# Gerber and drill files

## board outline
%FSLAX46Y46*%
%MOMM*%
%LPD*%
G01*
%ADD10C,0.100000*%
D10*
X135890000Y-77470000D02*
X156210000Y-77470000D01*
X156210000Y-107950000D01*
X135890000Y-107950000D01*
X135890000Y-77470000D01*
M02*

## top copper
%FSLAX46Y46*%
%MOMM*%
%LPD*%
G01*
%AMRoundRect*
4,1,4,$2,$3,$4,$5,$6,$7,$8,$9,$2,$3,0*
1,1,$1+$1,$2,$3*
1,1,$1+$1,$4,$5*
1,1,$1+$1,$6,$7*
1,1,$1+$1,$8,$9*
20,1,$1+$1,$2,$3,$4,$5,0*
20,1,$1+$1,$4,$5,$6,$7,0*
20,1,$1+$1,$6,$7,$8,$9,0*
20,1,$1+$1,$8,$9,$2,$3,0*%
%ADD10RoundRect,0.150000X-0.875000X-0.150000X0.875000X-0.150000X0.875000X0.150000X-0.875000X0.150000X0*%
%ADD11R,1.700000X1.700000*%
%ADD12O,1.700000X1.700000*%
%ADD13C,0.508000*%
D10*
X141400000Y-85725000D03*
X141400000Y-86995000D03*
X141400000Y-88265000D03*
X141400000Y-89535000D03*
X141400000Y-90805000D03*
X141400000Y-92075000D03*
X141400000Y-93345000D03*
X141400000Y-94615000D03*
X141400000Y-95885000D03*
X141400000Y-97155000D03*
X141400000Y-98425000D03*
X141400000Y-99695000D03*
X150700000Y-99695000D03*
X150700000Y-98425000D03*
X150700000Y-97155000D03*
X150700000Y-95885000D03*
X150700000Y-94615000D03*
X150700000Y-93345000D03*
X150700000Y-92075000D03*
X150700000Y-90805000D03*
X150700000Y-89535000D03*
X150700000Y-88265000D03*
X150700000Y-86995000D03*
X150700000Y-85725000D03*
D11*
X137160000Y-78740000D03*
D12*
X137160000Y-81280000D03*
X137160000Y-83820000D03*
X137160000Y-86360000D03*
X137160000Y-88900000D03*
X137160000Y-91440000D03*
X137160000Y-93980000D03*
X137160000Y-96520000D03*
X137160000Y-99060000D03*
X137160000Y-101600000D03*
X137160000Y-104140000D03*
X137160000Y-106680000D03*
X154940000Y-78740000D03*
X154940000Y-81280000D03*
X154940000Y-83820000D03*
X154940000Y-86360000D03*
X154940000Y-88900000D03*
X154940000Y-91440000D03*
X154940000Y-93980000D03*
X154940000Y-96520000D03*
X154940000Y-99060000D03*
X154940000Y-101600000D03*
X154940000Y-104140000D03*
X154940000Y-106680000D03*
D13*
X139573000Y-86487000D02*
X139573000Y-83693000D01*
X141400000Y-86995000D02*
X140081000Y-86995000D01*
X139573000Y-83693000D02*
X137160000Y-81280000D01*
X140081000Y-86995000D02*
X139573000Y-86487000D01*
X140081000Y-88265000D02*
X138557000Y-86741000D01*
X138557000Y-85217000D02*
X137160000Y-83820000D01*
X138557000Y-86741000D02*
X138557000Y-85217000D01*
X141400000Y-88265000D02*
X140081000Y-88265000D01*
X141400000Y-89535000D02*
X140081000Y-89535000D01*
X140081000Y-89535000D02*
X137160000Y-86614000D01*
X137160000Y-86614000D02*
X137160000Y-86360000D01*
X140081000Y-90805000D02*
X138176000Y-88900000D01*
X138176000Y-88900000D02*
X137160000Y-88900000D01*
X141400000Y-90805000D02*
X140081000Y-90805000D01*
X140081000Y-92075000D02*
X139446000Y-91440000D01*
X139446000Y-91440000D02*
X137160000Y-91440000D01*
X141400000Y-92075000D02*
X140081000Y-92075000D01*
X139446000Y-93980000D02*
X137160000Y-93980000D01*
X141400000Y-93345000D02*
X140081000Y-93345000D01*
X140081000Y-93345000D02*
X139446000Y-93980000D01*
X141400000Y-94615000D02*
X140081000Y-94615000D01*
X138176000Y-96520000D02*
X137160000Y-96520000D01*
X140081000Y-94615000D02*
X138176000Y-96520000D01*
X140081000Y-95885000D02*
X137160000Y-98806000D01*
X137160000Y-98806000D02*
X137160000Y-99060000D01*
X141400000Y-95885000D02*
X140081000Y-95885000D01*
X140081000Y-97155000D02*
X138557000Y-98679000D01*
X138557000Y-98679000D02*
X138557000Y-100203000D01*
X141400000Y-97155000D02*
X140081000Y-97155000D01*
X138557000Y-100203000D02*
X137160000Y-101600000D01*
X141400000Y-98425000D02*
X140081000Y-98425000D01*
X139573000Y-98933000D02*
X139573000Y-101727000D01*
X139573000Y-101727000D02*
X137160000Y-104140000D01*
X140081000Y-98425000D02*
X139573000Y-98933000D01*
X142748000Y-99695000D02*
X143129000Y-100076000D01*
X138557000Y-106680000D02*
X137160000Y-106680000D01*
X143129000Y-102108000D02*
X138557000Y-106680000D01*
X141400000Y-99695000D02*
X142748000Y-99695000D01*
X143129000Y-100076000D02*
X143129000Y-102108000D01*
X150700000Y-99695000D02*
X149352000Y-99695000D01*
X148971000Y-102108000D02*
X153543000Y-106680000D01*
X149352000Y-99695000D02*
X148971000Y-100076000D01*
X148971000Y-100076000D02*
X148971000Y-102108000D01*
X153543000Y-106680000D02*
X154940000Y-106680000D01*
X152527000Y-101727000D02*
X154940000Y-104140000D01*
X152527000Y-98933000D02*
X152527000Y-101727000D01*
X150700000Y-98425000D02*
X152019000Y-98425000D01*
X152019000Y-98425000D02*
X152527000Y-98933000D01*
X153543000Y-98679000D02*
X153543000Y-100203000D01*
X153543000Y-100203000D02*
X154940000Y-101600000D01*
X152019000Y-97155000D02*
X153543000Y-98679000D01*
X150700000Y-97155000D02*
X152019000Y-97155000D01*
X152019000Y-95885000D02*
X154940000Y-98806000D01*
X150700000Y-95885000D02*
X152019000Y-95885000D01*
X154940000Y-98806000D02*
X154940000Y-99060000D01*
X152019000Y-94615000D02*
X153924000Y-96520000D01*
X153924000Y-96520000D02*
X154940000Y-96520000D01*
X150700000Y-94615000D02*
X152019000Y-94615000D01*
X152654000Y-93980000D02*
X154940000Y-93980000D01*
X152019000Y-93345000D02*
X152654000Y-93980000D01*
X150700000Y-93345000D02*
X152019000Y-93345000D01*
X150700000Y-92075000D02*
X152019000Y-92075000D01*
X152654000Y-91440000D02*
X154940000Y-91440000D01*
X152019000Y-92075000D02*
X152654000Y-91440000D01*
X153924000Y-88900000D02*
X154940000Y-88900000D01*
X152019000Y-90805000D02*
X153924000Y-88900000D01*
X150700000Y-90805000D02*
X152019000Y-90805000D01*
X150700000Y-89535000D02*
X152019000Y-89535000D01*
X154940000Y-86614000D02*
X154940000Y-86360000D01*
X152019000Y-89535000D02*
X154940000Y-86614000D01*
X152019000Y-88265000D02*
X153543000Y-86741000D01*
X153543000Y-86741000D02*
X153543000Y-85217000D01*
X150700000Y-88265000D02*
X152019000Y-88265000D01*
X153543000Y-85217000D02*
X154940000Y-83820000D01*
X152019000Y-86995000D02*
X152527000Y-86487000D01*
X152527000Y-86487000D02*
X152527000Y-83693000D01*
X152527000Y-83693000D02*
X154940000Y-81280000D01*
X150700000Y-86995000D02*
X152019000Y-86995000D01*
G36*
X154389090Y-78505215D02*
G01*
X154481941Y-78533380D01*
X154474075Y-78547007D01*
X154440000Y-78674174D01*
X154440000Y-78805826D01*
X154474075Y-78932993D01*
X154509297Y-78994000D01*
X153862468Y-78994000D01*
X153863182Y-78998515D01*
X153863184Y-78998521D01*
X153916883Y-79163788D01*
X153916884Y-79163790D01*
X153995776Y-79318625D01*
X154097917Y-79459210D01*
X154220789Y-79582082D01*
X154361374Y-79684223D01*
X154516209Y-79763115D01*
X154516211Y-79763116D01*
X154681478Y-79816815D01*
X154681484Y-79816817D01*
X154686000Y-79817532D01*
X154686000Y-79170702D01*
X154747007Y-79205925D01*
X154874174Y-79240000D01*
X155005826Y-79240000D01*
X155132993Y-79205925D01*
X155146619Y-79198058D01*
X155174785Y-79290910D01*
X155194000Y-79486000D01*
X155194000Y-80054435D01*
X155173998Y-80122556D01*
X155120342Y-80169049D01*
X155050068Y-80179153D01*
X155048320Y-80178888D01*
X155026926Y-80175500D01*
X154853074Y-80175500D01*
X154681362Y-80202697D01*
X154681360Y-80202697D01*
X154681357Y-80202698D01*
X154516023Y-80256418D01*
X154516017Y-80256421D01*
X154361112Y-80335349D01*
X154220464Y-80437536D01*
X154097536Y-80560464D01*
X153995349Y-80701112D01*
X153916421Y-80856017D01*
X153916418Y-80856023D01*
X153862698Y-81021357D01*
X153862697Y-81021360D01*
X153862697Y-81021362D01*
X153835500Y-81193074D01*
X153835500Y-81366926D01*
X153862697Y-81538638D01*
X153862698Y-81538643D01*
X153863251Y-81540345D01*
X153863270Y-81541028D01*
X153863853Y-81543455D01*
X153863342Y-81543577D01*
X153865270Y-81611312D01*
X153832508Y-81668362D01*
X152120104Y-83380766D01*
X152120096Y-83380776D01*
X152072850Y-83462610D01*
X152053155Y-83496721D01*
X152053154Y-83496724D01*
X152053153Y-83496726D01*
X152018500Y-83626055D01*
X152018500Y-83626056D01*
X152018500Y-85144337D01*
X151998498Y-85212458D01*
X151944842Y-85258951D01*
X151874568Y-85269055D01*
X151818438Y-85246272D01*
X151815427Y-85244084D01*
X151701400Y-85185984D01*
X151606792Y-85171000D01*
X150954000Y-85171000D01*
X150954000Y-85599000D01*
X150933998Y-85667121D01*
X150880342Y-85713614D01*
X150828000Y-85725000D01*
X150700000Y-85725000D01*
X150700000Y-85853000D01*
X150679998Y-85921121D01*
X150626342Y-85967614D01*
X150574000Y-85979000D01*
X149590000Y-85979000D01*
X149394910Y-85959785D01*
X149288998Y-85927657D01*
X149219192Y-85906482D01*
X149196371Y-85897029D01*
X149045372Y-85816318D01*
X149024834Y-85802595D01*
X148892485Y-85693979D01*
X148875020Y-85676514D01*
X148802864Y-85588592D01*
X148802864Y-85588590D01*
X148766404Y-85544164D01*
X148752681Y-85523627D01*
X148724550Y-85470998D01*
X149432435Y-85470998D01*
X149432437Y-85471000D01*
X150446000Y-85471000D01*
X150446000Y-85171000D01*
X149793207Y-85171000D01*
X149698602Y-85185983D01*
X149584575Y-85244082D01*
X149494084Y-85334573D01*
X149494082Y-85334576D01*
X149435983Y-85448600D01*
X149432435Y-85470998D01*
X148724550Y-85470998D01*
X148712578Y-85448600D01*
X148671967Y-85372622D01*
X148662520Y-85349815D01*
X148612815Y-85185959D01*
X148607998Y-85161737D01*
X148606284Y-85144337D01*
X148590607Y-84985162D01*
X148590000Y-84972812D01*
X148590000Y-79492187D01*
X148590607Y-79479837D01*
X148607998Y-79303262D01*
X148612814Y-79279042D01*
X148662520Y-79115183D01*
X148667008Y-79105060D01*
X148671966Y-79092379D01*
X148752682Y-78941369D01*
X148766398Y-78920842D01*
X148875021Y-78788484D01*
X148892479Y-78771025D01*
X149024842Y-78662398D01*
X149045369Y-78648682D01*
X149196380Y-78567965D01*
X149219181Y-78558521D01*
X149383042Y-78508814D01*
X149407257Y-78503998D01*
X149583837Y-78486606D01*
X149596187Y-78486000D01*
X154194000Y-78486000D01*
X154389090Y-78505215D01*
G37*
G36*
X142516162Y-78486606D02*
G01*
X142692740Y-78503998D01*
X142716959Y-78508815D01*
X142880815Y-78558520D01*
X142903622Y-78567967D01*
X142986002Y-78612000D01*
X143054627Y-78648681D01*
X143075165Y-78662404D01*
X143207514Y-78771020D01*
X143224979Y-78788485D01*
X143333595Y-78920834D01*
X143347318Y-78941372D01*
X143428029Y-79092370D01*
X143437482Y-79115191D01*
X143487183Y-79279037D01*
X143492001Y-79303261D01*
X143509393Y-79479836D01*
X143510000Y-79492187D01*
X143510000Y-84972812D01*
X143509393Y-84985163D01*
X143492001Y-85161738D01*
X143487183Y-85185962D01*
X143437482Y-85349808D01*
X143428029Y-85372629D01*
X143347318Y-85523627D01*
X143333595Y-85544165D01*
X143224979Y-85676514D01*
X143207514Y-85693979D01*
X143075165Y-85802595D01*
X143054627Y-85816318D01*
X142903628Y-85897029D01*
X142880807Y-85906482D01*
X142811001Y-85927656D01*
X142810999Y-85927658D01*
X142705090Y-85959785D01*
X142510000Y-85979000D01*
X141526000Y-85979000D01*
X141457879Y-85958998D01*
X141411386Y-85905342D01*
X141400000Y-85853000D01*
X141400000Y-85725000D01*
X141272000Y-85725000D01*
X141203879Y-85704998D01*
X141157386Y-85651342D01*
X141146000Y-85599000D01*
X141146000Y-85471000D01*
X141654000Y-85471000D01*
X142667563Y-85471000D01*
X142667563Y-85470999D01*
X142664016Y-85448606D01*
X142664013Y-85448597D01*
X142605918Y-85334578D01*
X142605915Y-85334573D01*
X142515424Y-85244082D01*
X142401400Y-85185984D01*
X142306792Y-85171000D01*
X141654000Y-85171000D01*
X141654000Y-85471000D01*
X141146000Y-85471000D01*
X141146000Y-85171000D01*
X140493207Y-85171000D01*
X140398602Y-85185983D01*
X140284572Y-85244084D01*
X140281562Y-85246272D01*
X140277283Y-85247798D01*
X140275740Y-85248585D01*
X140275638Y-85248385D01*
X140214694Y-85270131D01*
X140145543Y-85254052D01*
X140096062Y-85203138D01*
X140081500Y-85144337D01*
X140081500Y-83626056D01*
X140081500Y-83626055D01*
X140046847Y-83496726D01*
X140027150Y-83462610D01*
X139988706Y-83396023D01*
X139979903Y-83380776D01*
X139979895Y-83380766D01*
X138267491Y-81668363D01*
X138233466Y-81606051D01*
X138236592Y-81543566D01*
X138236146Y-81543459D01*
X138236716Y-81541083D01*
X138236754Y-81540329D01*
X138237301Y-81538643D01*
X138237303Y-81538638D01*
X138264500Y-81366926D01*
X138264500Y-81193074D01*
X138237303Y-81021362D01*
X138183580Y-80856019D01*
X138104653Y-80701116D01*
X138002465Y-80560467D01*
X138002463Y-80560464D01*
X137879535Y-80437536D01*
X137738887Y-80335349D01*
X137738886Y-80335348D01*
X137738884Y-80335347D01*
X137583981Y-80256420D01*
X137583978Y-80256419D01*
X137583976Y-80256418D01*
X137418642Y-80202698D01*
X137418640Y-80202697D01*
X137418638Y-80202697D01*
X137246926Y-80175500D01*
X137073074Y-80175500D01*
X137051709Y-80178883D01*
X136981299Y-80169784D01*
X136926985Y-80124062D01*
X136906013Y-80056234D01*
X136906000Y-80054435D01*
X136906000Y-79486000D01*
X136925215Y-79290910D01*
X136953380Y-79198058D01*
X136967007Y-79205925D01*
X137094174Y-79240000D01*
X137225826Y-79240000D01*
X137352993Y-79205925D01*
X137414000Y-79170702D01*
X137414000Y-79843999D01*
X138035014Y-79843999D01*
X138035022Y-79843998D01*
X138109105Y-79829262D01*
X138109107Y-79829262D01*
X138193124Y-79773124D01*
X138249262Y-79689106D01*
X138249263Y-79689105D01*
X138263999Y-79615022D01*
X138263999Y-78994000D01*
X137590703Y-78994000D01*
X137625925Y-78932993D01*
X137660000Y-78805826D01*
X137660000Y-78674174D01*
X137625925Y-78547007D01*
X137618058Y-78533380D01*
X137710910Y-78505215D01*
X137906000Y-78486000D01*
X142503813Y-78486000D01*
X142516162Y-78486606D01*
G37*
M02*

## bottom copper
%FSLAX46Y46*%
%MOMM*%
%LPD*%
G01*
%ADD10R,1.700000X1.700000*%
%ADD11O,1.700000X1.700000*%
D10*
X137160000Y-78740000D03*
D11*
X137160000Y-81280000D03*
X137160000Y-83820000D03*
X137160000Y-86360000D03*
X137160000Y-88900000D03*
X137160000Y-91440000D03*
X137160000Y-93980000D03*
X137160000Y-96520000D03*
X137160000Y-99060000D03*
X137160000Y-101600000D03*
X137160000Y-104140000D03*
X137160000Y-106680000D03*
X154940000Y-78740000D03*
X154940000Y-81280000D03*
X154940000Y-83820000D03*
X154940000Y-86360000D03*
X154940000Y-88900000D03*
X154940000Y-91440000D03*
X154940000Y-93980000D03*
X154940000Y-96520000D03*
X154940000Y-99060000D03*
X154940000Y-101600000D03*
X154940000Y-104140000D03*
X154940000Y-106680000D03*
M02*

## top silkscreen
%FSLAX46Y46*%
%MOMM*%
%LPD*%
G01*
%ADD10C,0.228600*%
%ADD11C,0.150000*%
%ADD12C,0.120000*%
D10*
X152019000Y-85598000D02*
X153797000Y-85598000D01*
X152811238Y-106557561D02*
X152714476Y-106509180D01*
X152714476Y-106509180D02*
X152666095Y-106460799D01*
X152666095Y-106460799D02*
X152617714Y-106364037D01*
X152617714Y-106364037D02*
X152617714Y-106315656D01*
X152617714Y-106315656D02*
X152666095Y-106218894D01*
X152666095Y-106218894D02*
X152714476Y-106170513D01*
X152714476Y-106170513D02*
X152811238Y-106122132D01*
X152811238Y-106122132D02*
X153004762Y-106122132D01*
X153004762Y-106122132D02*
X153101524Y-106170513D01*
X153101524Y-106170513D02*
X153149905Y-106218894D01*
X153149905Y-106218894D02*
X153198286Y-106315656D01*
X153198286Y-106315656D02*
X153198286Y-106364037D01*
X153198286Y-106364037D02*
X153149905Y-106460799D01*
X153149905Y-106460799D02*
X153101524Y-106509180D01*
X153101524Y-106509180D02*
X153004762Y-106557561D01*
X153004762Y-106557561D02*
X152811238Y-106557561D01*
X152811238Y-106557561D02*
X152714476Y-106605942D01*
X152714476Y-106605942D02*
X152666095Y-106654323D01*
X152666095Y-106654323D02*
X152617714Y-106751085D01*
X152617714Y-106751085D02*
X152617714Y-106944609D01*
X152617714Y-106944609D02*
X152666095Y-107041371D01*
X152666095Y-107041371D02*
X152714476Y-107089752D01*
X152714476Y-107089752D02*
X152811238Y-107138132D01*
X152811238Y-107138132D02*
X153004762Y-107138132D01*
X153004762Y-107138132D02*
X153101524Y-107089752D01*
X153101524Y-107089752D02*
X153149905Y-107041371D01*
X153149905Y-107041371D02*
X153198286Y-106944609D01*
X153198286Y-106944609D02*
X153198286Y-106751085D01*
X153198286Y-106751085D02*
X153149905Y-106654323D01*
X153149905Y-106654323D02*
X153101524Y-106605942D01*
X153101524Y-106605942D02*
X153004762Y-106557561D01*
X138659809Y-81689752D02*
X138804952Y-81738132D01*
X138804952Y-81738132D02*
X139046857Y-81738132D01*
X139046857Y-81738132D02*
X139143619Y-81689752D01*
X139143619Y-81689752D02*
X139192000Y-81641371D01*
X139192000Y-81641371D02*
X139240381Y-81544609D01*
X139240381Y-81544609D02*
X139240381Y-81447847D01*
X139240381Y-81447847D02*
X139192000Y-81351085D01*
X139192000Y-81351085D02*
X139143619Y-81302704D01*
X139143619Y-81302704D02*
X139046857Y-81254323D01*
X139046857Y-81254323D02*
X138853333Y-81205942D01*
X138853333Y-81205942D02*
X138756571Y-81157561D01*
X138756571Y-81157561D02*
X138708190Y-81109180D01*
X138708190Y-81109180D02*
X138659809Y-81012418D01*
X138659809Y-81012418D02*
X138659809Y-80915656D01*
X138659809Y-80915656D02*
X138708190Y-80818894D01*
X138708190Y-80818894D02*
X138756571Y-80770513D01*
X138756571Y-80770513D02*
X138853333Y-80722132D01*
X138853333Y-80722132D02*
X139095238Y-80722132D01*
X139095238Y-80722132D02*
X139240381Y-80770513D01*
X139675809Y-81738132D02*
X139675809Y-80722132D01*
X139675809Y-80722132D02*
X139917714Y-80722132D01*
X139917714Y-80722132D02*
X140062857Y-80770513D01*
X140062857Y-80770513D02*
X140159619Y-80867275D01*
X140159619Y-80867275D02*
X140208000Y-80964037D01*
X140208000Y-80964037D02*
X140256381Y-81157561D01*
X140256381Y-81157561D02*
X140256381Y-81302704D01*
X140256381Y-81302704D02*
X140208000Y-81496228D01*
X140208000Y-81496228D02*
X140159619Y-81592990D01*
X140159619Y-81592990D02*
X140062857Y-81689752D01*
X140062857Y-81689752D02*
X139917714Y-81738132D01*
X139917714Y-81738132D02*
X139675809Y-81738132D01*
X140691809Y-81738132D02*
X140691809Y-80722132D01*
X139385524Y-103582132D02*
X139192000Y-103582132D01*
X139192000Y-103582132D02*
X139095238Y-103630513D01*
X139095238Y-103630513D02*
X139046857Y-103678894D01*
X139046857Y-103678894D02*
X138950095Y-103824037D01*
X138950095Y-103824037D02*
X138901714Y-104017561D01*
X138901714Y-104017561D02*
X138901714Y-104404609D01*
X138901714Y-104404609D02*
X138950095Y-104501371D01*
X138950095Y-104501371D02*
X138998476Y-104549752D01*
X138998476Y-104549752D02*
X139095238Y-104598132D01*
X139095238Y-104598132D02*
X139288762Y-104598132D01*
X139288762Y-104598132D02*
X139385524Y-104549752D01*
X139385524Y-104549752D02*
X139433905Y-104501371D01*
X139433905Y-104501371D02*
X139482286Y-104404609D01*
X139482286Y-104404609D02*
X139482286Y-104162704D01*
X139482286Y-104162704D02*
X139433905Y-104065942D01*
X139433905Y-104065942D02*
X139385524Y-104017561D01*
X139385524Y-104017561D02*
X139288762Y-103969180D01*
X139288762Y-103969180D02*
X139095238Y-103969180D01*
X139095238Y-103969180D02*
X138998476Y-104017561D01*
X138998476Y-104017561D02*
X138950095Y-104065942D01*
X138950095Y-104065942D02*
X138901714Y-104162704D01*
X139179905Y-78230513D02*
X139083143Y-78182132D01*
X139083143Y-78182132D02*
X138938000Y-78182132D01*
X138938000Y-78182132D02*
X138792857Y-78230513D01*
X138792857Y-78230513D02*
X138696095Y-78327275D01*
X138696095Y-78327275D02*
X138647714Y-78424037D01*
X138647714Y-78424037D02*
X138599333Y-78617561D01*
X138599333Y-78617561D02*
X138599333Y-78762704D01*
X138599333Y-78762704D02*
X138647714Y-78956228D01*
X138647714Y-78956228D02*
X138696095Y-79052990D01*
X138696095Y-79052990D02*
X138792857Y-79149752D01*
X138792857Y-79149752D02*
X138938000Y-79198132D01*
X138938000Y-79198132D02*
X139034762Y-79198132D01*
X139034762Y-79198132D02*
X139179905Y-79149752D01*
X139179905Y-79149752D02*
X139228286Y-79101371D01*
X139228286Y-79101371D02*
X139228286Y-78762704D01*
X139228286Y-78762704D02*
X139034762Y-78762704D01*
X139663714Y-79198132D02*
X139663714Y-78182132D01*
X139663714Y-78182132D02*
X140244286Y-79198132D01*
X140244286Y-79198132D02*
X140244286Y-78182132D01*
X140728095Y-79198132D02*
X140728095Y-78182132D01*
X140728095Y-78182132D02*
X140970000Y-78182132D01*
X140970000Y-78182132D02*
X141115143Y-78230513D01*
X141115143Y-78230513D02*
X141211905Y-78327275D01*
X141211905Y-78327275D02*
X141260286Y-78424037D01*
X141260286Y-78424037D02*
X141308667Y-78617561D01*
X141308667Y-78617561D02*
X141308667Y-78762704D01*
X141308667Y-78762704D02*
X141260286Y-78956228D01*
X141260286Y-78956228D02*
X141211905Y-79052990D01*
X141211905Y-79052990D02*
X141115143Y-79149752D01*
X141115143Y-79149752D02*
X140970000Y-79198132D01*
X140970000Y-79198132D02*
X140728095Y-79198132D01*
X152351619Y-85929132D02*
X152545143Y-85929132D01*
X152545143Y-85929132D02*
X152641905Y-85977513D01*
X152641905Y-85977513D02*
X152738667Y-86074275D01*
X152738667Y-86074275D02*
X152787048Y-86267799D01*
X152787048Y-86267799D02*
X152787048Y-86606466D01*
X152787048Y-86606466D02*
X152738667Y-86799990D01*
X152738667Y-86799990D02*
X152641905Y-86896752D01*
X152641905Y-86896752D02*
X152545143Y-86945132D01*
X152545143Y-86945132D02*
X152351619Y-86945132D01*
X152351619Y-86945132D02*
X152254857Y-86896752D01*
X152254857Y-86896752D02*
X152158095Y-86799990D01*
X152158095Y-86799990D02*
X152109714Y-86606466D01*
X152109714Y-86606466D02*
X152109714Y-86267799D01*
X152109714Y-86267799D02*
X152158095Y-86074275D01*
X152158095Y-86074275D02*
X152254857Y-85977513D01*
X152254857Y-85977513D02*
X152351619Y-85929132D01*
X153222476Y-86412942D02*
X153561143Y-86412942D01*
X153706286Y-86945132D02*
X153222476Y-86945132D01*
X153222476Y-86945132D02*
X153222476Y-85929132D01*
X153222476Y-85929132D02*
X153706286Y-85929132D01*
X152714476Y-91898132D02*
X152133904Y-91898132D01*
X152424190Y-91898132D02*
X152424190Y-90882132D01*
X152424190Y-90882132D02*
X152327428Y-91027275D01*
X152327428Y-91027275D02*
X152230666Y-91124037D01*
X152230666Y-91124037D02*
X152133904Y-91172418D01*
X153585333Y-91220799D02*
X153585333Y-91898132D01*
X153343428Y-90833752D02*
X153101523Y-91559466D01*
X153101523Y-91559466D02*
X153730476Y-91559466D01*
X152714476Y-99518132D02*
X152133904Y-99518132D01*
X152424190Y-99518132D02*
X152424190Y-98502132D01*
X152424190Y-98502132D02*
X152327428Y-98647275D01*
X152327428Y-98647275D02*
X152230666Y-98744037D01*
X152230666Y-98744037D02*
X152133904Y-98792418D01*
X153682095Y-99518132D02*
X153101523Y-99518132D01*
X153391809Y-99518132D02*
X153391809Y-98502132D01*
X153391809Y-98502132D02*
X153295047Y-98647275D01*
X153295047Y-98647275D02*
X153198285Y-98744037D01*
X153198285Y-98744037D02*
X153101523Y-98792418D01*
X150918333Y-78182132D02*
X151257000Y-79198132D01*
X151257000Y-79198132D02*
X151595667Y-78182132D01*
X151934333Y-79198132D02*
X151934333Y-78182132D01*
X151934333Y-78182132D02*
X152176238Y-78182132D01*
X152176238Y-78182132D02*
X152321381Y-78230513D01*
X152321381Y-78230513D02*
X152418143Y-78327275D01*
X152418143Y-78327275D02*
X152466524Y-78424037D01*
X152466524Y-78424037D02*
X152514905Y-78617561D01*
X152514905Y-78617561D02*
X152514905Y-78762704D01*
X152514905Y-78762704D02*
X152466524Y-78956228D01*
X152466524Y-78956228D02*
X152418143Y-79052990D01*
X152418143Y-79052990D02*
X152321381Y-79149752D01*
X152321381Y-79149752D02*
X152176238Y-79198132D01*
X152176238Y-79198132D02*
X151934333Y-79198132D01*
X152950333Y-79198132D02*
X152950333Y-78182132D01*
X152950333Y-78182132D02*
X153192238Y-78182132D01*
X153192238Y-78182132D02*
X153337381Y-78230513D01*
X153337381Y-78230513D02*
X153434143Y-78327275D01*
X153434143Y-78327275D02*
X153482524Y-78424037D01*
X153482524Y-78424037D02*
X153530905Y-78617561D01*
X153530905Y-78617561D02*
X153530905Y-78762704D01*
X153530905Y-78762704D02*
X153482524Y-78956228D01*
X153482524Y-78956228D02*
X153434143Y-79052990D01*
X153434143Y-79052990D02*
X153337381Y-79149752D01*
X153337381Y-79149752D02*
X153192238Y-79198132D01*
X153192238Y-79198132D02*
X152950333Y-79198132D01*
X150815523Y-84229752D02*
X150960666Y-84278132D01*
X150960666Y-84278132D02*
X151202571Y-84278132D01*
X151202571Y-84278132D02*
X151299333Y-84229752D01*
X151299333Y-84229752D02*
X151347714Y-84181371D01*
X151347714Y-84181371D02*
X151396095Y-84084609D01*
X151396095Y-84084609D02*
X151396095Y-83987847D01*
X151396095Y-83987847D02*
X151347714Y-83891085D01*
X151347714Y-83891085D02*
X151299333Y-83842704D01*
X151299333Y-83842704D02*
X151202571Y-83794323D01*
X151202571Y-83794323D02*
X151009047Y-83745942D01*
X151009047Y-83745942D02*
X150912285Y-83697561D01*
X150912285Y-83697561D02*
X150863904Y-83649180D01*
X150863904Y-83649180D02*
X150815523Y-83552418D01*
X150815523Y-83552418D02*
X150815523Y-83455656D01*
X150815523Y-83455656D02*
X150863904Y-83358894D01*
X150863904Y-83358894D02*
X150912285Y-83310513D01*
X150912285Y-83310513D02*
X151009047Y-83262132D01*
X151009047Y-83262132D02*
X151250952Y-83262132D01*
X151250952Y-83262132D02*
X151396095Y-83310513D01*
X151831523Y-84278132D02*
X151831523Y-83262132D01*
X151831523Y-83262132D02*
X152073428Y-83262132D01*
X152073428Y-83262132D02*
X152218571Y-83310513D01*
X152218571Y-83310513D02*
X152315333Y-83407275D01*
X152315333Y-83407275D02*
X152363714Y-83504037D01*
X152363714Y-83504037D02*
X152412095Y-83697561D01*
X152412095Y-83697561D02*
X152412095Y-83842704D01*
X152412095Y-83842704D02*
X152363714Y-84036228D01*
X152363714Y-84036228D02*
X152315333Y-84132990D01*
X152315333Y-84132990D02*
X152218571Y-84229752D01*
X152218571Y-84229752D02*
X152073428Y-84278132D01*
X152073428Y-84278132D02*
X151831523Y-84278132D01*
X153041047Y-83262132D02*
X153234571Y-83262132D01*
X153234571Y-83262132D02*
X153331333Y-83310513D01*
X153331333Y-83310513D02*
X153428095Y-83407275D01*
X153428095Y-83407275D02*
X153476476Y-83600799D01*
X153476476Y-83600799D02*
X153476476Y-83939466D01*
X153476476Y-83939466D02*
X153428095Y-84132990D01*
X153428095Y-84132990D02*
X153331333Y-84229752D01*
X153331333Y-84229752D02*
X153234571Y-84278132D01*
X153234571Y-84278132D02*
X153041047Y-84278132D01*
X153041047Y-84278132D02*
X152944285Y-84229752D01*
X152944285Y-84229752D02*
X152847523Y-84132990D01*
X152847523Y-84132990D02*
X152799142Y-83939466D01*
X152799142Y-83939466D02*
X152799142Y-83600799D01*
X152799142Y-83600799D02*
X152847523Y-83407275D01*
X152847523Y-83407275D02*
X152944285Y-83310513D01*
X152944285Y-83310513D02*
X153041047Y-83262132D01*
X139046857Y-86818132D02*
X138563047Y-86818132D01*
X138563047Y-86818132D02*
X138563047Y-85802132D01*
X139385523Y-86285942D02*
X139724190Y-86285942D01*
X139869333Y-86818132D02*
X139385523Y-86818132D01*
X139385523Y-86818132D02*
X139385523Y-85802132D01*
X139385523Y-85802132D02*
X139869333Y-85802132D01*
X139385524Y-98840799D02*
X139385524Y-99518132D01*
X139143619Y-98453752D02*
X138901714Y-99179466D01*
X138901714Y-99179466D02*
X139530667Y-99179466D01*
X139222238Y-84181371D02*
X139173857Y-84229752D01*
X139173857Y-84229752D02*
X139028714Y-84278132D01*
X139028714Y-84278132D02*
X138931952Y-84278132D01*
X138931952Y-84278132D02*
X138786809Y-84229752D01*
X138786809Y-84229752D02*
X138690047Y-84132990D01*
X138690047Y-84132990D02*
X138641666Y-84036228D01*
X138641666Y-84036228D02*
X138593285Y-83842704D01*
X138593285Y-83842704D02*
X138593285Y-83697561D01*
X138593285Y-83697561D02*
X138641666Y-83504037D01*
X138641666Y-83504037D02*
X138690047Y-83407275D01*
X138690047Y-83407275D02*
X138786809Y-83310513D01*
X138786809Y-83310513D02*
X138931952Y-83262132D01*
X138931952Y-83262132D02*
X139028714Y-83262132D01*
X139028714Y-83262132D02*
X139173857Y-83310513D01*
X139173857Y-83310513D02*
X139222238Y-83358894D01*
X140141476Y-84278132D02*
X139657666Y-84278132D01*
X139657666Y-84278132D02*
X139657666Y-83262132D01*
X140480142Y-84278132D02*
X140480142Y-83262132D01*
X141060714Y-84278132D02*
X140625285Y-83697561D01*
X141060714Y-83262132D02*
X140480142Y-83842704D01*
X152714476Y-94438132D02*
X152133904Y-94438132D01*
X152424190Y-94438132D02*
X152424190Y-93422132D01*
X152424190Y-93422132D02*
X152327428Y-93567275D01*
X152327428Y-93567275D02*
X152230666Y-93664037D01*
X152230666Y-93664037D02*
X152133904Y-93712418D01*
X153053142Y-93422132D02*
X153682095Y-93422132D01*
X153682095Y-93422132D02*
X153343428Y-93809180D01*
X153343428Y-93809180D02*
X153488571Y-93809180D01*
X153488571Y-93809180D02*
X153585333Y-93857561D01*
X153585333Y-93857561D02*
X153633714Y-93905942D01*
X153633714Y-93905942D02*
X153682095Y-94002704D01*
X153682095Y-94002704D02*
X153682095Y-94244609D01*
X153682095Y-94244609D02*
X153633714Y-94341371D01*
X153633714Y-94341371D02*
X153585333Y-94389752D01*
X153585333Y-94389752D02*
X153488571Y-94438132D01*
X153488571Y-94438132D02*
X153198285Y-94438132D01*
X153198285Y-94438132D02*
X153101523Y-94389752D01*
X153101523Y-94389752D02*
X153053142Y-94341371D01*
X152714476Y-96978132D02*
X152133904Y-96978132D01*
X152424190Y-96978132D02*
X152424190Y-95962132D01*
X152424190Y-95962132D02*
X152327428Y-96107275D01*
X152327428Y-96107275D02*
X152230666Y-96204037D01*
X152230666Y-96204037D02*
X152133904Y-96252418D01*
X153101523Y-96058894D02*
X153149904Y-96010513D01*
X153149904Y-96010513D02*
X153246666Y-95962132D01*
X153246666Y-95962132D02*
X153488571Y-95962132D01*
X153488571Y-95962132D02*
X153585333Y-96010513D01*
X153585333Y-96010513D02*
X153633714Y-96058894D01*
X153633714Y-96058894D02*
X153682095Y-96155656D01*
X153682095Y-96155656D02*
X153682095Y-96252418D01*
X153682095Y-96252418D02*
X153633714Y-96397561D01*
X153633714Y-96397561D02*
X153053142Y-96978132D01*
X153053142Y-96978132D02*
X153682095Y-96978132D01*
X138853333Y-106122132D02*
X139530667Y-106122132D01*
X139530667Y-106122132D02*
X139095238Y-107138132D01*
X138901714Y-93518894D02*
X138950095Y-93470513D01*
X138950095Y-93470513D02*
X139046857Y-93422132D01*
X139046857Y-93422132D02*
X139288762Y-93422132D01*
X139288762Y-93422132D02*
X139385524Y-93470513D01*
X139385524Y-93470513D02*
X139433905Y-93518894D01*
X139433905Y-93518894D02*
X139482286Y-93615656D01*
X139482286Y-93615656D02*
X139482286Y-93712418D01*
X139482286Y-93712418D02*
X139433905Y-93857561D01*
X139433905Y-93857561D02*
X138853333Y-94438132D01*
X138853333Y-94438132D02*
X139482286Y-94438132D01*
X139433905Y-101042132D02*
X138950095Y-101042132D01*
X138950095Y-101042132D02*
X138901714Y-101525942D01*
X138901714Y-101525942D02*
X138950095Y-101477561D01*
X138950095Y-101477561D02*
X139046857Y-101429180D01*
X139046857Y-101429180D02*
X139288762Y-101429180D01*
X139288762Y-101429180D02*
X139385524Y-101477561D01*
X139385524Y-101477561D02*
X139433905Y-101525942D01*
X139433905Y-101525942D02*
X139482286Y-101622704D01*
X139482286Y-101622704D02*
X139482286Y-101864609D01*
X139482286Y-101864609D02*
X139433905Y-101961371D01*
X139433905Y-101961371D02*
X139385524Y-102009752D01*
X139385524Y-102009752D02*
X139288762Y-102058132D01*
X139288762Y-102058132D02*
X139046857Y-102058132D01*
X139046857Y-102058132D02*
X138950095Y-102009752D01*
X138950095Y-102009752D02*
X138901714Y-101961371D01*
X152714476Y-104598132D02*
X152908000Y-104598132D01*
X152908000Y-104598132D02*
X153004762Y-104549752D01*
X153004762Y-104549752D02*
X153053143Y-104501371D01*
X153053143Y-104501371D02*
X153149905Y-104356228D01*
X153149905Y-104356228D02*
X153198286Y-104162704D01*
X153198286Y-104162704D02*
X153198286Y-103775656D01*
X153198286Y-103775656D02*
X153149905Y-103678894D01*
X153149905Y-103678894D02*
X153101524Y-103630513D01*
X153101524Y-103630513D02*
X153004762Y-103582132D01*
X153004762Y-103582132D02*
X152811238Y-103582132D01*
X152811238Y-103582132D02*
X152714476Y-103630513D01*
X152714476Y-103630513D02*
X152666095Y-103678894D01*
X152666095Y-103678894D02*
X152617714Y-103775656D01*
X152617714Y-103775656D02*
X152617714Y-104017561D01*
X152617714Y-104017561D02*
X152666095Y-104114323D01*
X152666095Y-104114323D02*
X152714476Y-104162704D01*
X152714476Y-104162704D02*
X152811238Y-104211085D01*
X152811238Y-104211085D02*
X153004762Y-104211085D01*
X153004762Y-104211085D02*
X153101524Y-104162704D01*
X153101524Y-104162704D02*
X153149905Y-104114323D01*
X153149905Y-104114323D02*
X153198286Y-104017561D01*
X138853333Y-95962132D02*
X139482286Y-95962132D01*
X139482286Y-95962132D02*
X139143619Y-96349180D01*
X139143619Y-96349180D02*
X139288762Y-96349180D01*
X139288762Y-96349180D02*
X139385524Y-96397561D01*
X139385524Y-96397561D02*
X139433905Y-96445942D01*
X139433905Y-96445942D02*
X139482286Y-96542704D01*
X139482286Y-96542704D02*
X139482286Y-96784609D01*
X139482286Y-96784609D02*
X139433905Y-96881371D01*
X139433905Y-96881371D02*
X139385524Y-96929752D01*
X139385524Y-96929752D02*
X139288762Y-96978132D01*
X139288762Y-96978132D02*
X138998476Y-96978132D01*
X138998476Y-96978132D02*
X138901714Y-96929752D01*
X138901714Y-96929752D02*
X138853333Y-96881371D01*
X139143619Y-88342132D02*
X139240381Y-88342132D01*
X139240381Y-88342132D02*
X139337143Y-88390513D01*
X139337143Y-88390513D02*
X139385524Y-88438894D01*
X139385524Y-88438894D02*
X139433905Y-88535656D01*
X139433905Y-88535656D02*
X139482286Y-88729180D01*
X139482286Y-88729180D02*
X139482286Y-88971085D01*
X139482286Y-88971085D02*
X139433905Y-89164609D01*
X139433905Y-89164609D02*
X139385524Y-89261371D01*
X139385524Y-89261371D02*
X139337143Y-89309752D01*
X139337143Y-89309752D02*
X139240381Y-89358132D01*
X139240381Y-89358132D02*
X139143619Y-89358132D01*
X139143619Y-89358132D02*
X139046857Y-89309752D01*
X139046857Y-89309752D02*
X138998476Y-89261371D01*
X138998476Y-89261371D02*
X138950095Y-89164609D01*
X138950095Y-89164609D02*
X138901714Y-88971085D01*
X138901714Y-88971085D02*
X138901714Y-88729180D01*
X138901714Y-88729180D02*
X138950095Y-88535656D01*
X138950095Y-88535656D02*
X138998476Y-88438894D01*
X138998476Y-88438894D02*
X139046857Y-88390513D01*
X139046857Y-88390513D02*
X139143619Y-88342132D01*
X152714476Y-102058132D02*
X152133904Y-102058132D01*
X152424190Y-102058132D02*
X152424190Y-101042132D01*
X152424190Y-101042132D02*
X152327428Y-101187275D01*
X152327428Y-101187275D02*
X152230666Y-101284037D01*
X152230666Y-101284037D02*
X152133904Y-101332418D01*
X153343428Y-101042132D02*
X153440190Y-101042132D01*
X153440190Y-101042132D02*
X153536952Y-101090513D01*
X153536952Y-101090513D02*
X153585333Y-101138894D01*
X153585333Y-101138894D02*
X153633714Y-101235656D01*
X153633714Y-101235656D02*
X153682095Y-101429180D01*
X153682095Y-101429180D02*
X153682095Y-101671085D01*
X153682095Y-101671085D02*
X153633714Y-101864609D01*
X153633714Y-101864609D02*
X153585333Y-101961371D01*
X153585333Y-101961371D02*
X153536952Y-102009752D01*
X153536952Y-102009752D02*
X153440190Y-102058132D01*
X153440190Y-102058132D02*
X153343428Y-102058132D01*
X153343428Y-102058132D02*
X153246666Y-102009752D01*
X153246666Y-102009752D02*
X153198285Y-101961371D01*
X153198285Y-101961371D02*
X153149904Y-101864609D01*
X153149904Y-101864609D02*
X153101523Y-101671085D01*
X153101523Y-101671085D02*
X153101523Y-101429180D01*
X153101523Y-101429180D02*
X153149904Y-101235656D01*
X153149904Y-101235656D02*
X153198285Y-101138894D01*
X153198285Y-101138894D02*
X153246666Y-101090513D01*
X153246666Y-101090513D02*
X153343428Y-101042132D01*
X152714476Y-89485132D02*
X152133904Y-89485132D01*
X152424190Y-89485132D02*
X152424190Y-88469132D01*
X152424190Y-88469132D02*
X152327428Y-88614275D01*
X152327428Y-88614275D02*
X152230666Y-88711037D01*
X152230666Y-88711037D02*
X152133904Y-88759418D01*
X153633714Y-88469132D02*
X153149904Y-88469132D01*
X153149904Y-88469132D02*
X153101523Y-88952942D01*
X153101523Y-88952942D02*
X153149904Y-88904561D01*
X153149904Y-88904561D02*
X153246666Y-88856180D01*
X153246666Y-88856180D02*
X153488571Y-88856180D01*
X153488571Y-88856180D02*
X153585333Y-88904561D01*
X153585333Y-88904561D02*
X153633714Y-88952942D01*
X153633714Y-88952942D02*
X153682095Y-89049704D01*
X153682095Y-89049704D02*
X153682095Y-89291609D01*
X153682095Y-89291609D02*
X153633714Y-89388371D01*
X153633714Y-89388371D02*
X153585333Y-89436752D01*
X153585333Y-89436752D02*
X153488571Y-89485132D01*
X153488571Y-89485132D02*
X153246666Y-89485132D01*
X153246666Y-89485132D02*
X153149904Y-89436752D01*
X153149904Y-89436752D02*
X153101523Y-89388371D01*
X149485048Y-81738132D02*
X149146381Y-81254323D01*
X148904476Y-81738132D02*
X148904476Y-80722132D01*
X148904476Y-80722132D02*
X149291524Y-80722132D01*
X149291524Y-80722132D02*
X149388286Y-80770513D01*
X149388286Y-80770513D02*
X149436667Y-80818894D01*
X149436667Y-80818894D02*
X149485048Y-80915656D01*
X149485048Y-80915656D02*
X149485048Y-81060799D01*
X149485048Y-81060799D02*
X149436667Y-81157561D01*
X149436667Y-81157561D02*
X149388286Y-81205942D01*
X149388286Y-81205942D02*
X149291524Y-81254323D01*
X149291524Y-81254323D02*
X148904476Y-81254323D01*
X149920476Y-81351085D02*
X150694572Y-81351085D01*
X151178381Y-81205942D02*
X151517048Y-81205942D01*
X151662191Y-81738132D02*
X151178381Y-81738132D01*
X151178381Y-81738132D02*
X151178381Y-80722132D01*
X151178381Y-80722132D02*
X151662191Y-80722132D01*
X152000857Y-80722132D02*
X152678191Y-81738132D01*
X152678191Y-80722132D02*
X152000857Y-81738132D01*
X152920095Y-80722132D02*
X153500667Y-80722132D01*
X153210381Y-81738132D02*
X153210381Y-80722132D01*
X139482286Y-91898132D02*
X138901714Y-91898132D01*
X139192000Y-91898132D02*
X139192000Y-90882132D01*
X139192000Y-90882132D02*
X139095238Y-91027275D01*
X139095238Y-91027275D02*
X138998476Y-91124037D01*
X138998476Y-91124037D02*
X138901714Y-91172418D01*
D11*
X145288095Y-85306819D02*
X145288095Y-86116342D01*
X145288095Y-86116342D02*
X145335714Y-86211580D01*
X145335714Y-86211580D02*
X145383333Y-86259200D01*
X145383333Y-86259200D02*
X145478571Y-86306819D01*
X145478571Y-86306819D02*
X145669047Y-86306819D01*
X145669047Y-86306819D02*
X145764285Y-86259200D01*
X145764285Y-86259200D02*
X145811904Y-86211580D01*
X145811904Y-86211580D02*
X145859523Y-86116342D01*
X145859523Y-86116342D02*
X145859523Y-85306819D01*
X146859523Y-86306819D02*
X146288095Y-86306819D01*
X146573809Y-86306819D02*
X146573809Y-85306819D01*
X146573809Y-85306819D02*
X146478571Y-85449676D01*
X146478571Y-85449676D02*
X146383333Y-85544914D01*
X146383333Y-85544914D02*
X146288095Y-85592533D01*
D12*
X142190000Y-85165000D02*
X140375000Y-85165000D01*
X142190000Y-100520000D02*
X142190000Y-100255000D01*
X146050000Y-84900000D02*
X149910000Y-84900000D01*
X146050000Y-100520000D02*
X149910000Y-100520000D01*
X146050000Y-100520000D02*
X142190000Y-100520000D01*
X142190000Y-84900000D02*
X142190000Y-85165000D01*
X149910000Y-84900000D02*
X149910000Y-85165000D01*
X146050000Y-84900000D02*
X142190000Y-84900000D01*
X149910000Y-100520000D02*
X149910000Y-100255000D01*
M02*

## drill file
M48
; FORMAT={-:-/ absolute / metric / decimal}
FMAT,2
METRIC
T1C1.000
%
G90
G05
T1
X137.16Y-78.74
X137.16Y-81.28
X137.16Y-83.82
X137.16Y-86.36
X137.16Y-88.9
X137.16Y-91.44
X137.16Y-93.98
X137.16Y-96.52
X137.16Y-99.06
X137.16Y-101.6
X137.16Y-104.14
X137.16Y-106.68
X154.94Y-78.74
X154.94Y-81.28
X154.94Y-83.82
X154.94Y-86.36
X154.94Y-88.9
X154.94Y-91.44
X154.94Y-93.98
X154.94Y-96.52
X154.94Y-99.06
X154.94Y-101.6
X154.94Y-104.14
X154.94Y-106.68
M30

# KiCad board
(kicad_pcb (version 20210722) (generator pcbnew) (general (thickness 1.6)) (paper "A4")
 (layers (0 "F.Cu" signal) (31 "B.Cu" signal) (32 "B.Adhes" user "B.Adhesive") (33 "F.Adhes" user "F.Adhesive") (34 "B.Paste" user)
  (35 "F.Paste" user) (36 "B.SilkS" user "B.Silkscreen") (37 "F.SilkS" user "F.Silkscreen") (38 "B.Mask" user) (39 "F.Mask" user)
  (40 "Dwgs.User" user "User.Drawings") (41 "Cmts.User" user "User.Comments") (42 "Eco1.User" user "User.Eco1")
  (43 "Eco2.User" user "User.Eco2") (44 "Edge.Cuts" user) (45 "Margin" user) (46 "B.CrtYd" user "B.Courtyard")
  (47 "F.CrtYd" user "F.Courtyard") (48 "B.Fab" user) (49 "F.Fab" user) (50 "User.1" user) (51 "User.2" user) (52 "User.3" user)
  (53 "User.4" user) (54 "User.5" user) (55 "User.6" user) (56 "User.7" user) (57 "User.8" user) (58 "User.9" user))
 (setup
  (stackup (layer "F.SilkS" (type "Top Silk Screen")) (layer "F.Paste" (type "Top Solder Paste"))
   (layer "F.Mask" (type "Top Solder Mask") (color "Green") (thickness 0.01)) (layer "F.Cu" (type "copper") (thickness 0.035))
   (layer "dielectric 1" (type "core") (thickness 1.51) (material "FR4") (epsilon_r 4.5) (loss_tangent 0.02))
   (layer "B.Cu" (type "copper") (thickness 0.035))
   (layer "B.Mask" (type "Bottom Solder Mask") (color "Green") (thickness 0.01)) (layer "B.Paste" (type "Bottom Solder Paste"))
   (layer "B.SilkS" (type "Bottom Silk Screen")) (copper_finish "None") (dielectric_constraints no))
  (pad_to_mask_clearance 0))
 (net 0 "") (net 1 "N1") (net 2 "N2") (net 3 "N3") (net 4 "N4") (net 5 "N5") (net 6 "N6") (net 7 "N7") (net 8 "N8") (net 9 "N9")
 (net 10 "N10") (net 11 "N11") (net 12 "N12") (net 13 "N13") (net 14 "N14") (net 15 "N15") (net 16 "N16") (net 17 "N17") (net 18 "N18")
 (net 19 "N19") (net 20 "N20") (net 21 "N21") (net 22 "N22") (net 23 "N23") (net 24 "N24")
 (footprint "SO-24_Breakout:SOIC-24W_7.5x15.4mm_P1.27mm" (layer "F.Cu") (at 146.05 92.71)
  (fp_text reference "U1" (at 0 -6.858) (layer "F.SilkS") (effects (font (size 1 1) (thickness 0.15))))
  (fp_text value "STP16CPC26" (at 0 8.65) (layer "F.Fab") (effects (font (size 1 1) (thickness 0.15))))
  (fp_line (start -3.86 -7.545) (end -5.675 -7.545) (layer "F.SilkS") (width 0.12))
  (fp_line (start -3.86 7.81) (end -3.86 7.545) (layer "F.SilkS") (width 0.12))
  (fp_line (start 0 -7.81) (end 3.86 -7.81) (layer "F.SilkS") (width 0.12))
  (fp_line (start 0 7.81) (end 3.86 7.81) (layer "F.SilkS") (width 0.12))
  (fp_line (start 0 7.81) (end -3.86 7.81) (layer "F.SilkS") (width 0.12))
  (fp_line (start -3.86 -7.81) (end -3.86 -7.545) (layer "F.SilkS") (width 0.12))
  (fp_line (start 3.86 -7.81) (end 3.86 -7.545) (layer "F.SilkS") (width 0.12))
  (fp_line (start 0 -7.81) (end -3.86 -7.81) (layer "F.SilkS") (width 0.12))
  (fp_line (start 3.86 7.81) (end 3.86 7.545) (layer "F.SilkS") (width 0.12))
  (pad "1" smd roundrect locked (at -4.65 -6.985) (size 2.05 0.6) (layers "F.Cu" "F.Paste" "F.Mask") (roundrect_rratio 0.25) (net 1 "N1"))
  (pad "2" smd roundrect locked (at -4.65 -5.715) (size 2.05 0.6) (layers "F.Cu" "F.Paste" "F.Mask") (roundrect_rratio 0.25) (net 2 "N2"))
  (pad "3" smd roundrect locked (at -4.65 -4.445) (size 2.05 0.6) (layers "F.Cu" "F.Paste" "F.Mask") (roundrect_rratio 0.25) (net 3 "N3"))
  (pad "4" smd roundrect locked (at -4.65 -3.175) (size 2.05 0.6) (layers "F.Cu" "F.Paste" "F.Mask") (roundrect_rratio 0.25) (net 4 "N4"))
  (pad "5" smd roundrect locked (at -4.65 -1.905) (size 2.05 0.6) (layers "F.Cu" "F.Paste" "F.Mask") (roundrect_rratio 0.25) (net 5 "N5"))
  (pad "6" smd roundrect locked (at -4.65 -0.635) (size 2.05 0.6) (layers "F.Cu" "F.Paste" "F.Mask") (roundrect_rratio 0.25) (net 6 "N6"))
  (pad "7" smd roundrect locked (at -4.65 0.635) (size 2.05 0.6) (layers "F.Cu" "F.Paste" "F.Mask") (roundrect_rratio 0.25) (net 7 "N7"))
  (pad "8" smd roundrect locked (at -4.65 1.905) (size 2.05 0.6) (layers "F.Cu" "F.Paste" "F.Mask") (roundrect_rratio 0.25) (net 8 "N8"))
  (pad "9" smd roundrect locked (at -4.65 3.175) (size 2.05 0.6) (layers "F.Cu" "F.Paste" "F.Mask") (roundrect_rratio 0.25) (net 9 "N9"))
  (pad "10" smd roundrect locked (at -4.65 4.445) (size 2.05 0.6) (layers "F.Cu" "F.Paste" "F.Mask") (roundrect_rratio 0.25) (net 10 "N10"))
  (pad "11" smd roundrect locked (at -4.65 5.715) (size 2.05 0.6) (layers "F.Cu" "F.Paste" "F.Mask") (roundrect_rratio 0.25) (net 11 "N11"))
  (pad "12" smd roundrect locked (at -4.65 6.985) (size 2.05 0.6) (layers "F.Cu" "F.Paste" "F.Mask") (roundrect_rratio 0.25) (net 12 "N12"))
  (pad "13" smd roundrect locked (at 4.65 6.985) (size 2.05 0.6) (layers "F.Cu" "F.Paste" "F.Mask") (roundrect_rratio 0.25) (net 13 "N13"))
  (pad "14" smd roundrect locked (at 4.65 5.715) (size 2.05 0.6) (layers "F.Cu" "F.Paste" "F.Mask") (roundrect_rratio 0.25) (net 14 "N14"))
  (pad "15" smd roundrect locked (at 4.65 4.445) (size 2.05 0.6) (layers "F.Cu" "F.Paste" "F.Mask") (roundrect_rratio 0.25) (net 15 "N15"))
  (pad "16" smd roundrect locked (at 4.65 3.175) (size 2.05 0.6) (layers "F.Cu" "F.Paste" "F.Mask") (roundrect_rratio 0.25) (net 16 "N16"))
  (pad "17" smd roundrect locked (at 4.65 1.905) (size 2.05 0.6) (layers "F.Cu" "F.Paste" "F.Mask") (roundrect_rratio 0.25) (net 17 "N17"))
  (pad "18" smd roundrect locked (at 4.65 0.635) (size 2.05 0.6) (layers "F.Cu" "F.Paste" "F.Mask") (roundrect_rratio 0.25) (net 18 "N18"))
  (pad "19" smd roundrect locked (at 4.65 -0.635) (size 2.05 0.6) (layers "F.Cu" "F.Paste" "F.Mask") (roundrect_rratio 0.25) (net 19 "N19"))
  (pad "20" smd roundrect locked (at 4.65 -1.905) (size 2.05 0.6) (layers "F.Cu" "F.Paste" "F.Mask") (roundrect_rratio 0.25) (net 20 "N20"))
  (pad "21" smd roundrect locked (at 4.65 -3.175) (size 2.05 0.6) (layers "F.Cu" "F.Paste" "F.Mask") (roundrect_rratio 0.25) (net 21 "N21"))
  (pad "22" smd roundrect locked (at 4.65 -4.445) (size 2.05 0.6) (layers "F.Cu" "F.Paste" "F.Mask") (roundrect_rratio 0.25) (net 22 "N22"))
  (pad "23" smd roundrect locked (at 4.65 -5.715) (size 2.05 0.6) (layers "F.Cu" "F.Paste" "F.Mask") (roundrect_rratio 0.25) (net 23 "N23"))
  (pad "24" smd roundrect locked (at 4.65 -6.985) (size 2.05 0.6) (layers "F.Cu" "F.Paste" "F.Mask") (roundrect_rratio 0.25) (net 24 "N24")))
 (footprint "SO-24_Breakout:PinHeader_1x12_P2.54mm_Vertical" (layer "B.Cu") (at 137.16 78.74 180)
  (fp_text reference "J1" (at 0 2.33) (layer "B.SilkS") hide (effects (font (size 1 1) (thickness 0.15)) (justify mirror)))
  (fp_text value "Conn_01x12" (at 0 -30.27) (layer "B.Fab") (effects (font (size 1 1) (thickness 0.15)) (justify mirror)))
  (pad "1" thru_hole rect locked (at 0 0 180) (size 1.7 1.7) (drill 1) (layers *.Cu *.Mask) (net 1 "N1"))
  (pad "2" thru_hole oval locked (at 0 -2.54 180) (size 1.7 1.7) (drill 1) (layers *.Cu *.Mask) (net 2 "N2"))
  (pad "3" thru_hole oval locked (at 0 -5.08 180) (size 1.7 1.7) (drill 1) (layers *.Cu *.Mask) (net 3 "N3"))
  (pad "4" thru_hole oval locked (at 0 -7.62 180) (size 1.7 1.7) (drill 1) (layers *.Cu *.Mask) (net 4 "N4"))
  (pad "5" thru_hole oval locked (at 0 -10.16 180) (size 1.7 1.7) (drill 1) (layers *.Cu *.Mask) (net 5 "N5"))
  (pad "6" thru_hole oval locked (at 0 -12.7 180) (size 1.7 1.7) (drill 1) (layers *.Cu *.Mask) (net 6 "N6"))
  (pad "7" thru_hole oval locked (at 0 -15.24 180) (size 1.7 1.7) (drill 1) (layers *.Cu *.Mask) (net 7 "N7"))
  (pad "8" thru_hole oval locked (at 0 -17.78 180) (size 1.7 1.7) (drill 1) (layers *.Cu *.Mask) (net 8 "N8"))
  (pad "9" thru_hole oval locked (at 0 -20.32 180) (size 1.7 1.7) (drill 1) (layers *.Cu *.Mask) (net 9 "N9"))
  (pad "10" thru_hole oval locked (at 0 -22.86 180) (size 1.7 1.7) (drill 1) (layers *.Cu *.Mask) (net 10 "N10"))
  (pad "11" thru_hole oval locked (at 0 -25.4 180) (size 1.7 1.7) (drill 1) (layers *.Cu *.Mask) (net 11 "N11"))
  (pad "12" thru_hole oval locked (at 0 -27.94 180) (size 1.7 1.7) (drill 1) (layers *.Cu *.Mask) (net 12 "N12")))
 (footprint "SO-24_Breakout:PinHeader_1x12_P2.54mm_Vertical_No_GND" (layer "B.Cu") (at 154.94 78.74 180)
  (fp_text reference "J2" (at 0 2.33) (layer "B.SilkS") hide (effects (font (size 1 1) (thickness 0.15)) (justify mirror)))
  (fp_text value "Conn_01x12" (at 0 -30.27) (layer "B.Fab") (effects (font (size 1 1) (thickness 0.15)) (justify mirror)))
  (pad "1" thru_hole oval locked (at 0 0 180) (size 1.7 1.7) (drill 1) (layers *.Cu *.Mask) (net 24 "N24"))
  (pad "2" thru_hole oval locked (at 0 -2.54 180) (size 1.7 1.7) (drill 1) (layers *.Cu *.Mask) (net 23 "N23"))
  (pad "3" thru_hole oval locked (at 0 -5.08 180) (size 1.7 1.7) (drill 1) (layers *.Cu *.Mask) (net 22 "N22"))
  (pad "4" thru_hole oval locked (at 0 -7.62 180) (size 1.7 1.7) (drill 1) (layers *.Cu *.Mask) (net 21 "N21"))
  (pad "5" thru_hole oval locked (at 0 -10.16 180) (size 1.7 1.7) (drill 1) (layers *.Cu *.Mask) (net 20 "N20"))
  (pad "6" thru_hole oval locked (at 0 -12.7 180) (size 1.7 1.7) (drill 1) (layers *.Cu *.Mask) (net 19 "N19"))
  (pad "7" thru_hole oval locked (at 0 -15.24 180) (size 1.7 1.7) (drill 1) (layers *.Cu *.Mask) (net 18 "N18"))
  (pad "8" thru_hole oval locked (at 0 -17.78 180) (size 1.7 1.7) (drill 1) (layers *.Cu *.Mask) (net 17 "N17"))
  (pad "9" thru_hole oval locked (at 0 -20.32 180) (size 1.7 1.7) (drill 1) (layers *.Cu *.Mask) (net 16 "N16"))
  (pad "10" thru_hole oval locked (at 0 -22.86 180) (size 1.7 1.7) (drill 1) (layers *.Cu *.Mask) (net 15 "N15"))
  (pad "11" thru_hole oval locked (at 0 -25.4 180) (size 1.7 1.7) (drill 1) (layers *.Cu *.Mask) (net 14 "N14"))
  (pad "12" thru_hole oval locked (at 0 -27.94 180) (size 1.7 1.7) (drill 1) (layers *.Cu *.Mask) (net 13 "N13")))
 (gr_line (start 152.019 85.598) (end 153.797 85.598) (layer "F.SilkS") (width 0.2286))
 (gr_rect (start 135.89 77.47) (end 156.21 107.95) (layer "Edge.Cuts") (width 0.1) (fill none))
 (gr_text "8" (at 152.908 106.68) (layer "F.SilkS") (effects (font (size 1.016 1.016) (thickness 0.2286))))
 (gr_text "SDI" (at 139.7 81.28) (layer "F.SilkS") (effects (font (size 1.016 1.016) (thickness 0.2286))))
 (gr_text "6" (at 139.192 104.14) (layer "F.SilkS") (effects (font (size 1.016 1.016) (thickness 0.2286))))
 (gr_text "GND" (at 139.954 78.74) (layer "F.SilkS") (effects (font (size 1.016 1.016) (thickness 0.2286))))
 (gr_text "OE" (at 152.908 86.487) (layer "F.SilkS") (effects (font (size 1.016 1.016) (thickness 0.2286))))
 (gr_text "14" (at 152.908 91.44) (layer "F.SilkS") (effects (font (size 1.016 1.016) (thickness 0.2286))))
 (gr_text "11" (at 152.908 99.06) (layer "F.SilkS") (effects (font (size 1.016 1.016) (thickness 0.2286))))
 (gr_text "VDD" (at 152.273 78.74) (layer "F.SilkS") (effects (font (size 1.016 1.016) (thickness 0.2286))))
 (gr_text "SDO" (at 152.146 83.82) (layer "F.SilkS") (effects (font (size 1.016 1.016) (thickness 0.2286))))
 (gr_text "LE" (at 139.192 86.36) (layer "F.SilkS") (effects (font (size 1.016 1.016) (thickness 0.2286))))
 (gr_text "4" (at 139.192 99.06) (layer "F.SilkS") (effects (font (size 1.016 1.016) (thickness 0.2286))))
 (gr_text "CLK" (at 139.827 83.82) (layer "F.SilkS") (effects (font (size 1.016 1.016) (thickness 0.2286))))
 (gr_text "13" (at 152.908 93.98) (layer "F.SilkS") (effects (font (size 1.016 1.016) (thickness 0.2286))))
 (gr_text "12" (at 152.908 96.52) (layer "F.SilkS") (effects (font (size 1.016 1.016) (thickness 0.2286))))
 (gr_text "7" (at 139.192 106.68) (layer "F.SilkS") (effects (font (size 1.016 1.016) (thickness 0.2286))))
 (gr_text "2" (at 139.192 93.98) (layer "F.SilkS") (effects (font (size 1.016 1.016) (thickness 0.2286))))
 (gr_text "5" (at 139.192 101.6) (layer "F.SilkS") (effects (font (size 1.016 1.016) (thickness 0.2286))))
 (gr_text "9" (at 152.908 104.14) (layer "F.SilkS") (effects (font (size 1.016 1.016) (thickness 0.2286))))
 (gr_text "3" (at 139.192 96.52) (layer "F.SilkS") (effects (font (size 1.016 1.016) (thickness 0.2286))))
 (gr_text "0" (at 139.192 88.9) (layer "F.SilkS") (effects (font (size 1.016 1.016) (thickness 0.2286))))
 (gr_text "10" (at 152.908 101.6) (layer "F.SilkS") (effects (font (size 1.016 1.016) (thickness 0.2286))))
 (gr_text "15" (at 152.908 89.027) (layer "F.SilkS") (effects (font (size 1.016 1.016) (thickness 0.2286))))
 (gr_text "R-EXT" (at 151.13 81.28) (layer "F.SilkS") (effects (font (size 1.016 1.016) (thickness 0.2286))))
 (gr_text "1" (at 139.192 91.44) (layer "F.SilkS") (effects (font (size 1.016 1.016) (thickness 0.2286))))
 (segment (start 139.573 86.487) (end 139.573 83.693) (width 0.508) (layer "F.Cu") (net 2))
 (segment (start 141.4 86.995) (end 140.081 86.995) (width 0.508) (layer "F.Cu") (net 2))
 (segment (start 139.573 83.693) (end 137.16 81.28) (width 0.508) (layer "F.Cu") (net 2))
 (segment (start 140.081 86.995) (end 139.573 86.487) (width 0.508) (layer "F.Cu") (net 2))
 (segment (start 140.081 88.265) (end 138.557 86.741) (width 0.508) (layer "F.Cu") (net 3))
 (segment (start 138.557 85.217) (end 137.16 83.82) (width 0.508) (layer "F.Cu") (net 3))
 (segment (start 138.557 86.741) (end 138.557 85.217) (width 0.508) (layer "F.Cu") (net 3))
 (segment (start 141.4 88.265) (end 140.081 88.265) (width 0.508) (layer "F.Cu") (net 3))
 (segment (start 141.4 89.535) (end 140.081 89.535) (width 0.508) (layer "F.Cu") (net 4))
 (segment (start 140.081 89.535) (end 137.16 86.614) (width 0.508) (layer "F.Cu") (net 4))
 (segment (start 137.16 86.614) (end 137.16 86.36) (width 0.508) (layer "F.Cu") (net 4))
 (segment (start 140.081 90.805) (end 138.176 88.9) (width 0.508) (layer "F.Cu") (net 5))
 (segment (start 138.176 88.9) (end 137.16 88.9) (width 0.508) (layer "F.Cu") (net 5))
 (segment (start 141.4 90.805) (end 140.081 90.805) (width 0.508) (layer "F.Cu") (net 5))
 (segment (start 140.081 92.075) (end 139.446 91.44) (width 0.508) (layer "F.Cu") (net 6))
 (segment (start 139.446 91.44) (end 137.16 91.44) (width 0.508) (layer "F.Cu") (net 6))
 (segment (start 141.4 92.075) (end 140.081 92.075) (width 0.508) (layer "F.Cu") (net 6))
 (segment (start 139.446 93.98) (end 137.16 93.98) (width 0.508) (layer "F.Cu") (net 7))
 (segment (start 141.4 93.345) (end 140.081 93.345) (width 0.508) (layer "F.Cu") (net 7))
 (segment (start 140.081 93.345) (end 139.446 93.98) (width 0.508) (layer "F.Cu") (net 7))
 (segment (start 141.4 94.615) (end 140.081 94.615) (width 0.508) (layer "F.Cu") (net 8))
 (segment (start 138.176 96.52) (end 137.16 96.52) (width 0.508) (layer "F.Cu") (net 8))
 (segment (start 140.081 94.615) (end 138.176 96.52) (width 0.508) (layer "F.Cu") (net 8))
 (segment (start 140.081 95.885) (end 137.16 98.806) (width 0.508) (layer "F.Cu") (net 9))
 (segment (start 137.16 98.806) (end 137.16 99.06) (width 0.508) (layer "F.Cu") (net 9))
 (segment (start 141.4 95.885) (end 140.081 95.885) (width 0.508) (layer "F.Cu") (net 9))
 (segment (start 140.081 97.155) (end 138.557 98.679) (width 0.508) (layer "F.Cu") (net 10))
 (segment (start 138.557 98.679) (end 138.557 100.203) (width 0.508) (layer "F.Cu") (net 10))
 (segment (start 141.4 97.155) (end 140.081 97.155) (width 0.508) (layer "F.Cu") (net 10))
 (segment (start 138.557 100.203) (end 137.16 101.6) (width 0.508) (layer "F.Cu") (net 10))
 (segment (start 141.4 98.425) (end 140.081 98.425) (width 0.508) (layer "F.Cu") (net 11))
 (segment (start 139.573 98.933) (end 139.573 101.727) (width 0.508) (layer "F.Cu") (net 11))
 (segment (start 139.573 101.727) (end 137.16 104.14) (width 0.508) (layer "F.Cu") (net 11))
 (segment (start 140.081 98.425) (end 139.573 98.933) (width 0.508) (layer "F.Cu") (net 11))
 (segment (start 142.748 99.695) (end 143.129 100.076) (width 0.508) (layer "F.Cu") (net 12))
 (segment (start 138.557 106.68) (end 137.16 106.68) (width 0.508) (layer "F.Cu") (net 12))
 (segment (start 143.129 102.108) (end 138.557 106.68) (width 0.508) (layer "F.Cu") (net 12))
 (segment (start 141.4 99.695) (end 142.748 99.695) (width 0.508) (layer "F.Cu") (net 12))
 (segment (start 143.129 100.076) (end 143.129 102.108) (width 0.508) (layer "F.Cu") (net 12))
 (segment (start 150.7 99.695) (end 149.352 99.695) (width 0.508) (layer "F.Cu") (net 13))
 (segment (start 148.971 102.108) (end 153.543 106.68) (width 0.508) (layer "F.Cu") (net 13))
 (segment (start 149.352 99.695) (end 148.971 100.076) (width 0.508) (layer "F.Cu") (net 13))
 (segment (start 148.971 100.076) (end 148.971 102.108) (width 0.508) (layer "F.Cu") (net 13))
 (segment (start 153.543 106.68) (end 154.94 106.68) (width 0.508) (layer "F.Cu") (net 13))
 (segment (start 152.527 101.727) (end 154.94 104.14) (width 0.508) (layer "F.Cu") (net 14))
 (segment (start 152.527 98.933) (end 152.527 101.727) (width 0.508) (layer "F.Cu") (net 14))
 (segment (start 150.7 98.425) (end 152.019 98.425) (width 0.508) (layer "F.Cu") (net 14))
 (segment (start 152.019 98.425) (end 152.527 98.933) (width 0.508) (layer "F.Cu") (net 14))
 (segment (start 153.543 98.679) (end 153.543 100.203) (width 0.508) (layer "F.Cu") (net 15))
 (segment (start 153.543 100.203) (end 154.94 101.6) (width 0.508) (layer "F.Cu") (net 15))
 (segment (start 152.019 97.155) (end 153.543 98.679) (width 0.508) (layer "F.Cu") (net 15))
 (segment (start 150.7 97.155) (end 152.019 97.155) (width 0.508) (layer "F.Cu") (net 15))
 (segment (start 152.019 95.885) (end 154.94 98.806) (width 0.508) (layer "F.Cu") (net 16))
 (segment (start 150.7 95.885) (end 152.019 95.885) (width 0.508) (layer "F.Cu") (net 16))
 (segment (start 154.94 98.806) (end 154.94 99.06) (width 0.508) (layer "F.Cu") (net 16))
 (segment (start 152.019 94.615) (end 153.924 96.52) (width 0.508) (layer "F.Cu") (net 17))
 (segment (start 153.924 96.52) (end 154.94 96.52) (width 0.508) (layer "F.Cu") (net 17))
 (segment (start 150.7 94.615) (end 152.019 94.615) (width 0.508) (layer "F.Cu") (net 17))
 (segment (start 152.654 93.98) (end 154.94 93.98) (width 0.508) (layer "F.Cu") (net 18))
 (segment (start 152.019 93.345) (end 152.654 93.98) (width 0.508) (layer "F.Cu") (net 18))
 (segment (start 150.7 93.345) (end 152.019 93.345) (width 0.508) (layer "F.Cu") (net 18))
 (segment (start 150.7 92.075) (end 152.019 92.075) (width 0.508) (layer "F.Cu") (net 19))
 (segment (start 152.654 91.44) (end 154.94 91.44) (width 0.508) (layer "F.Cu") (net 19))
 (segment (start 152.019 92.075) (end 152.654 91.44) (width 0.508) (layer "F.Cu") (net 19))
 (segment (start 153.924 88.9) (end 154.94 88.9) (width 0.508) (layer "F.Cu") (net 20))
 (segment (start 152.019 90.805) (end 153.924 88.9) (width 0.508) (layer "F.Cu") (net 20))
 (segment (start 150.7 90.805) (end 152.019 90.805) (width 0.508) (layer "F.Cu") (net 20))
 (segment (start 150.7 89.535) (end 152.019 89.535) (width 0.508) (layer "F.Cu") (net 21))
 (segment (start 154.94 86.614) (end 154.94 86.36) (width 0.508) (layer "F.Cu") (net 21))
 (segment (start 152.019 89.535) (end 154.94 86.614) (width 0.508) (layer "F.Cu") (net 21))
 (segment (start 152.019 88.265) (end 153.543 86.741) (width 0.508) (layer "F.Cu") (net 22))
 (segment (start 153.543 86.741) (end 153.543 85.217) (width 0.508) (layer "F.Cu") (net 22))
 (segment (start 150.7 88.265) (end 152.019 88.265) (width 0.508) (layer "F.Cu") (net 22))
 (segment (start 153.543 85.217) (end 154.94 83.82) (width 0.508) (layer "F.Cu") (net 22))
 (segment (start 152.019 86.995) (end 152.527 86.487) (width 0.508) (layer "F.Cu") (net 23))
 (segment (start 152.527 86.487) (end 152.527 83.693) (width 0.508) (layer "F.Cu") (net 23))
 (segment (start 152.527 83.693) (end 154.94 81.28) (width 0.508) (layer "F.Cu") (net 23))
 (segment (start 150.7 86.995) (end 152.019 86.995) (width 0.508) (layer "F.Cu") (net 23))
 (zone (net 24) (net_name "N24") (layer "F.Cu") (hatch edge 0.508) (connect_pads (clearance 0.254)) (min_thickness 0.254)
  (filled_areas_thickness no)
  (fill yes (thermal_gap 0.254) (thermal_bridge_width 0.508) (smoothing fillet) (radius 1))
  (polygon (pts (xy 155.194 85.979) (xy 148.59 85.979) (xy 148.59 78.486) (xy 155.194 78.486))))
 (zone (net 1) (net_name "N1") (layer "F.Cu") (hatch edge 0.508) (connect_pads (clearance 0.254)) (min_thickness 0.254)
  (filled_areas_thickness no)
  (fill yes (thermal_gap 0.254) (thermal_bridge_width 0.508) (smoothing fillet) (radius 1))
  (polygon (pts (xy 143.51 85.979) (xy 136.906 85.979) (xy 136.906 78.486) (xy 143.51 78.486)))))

